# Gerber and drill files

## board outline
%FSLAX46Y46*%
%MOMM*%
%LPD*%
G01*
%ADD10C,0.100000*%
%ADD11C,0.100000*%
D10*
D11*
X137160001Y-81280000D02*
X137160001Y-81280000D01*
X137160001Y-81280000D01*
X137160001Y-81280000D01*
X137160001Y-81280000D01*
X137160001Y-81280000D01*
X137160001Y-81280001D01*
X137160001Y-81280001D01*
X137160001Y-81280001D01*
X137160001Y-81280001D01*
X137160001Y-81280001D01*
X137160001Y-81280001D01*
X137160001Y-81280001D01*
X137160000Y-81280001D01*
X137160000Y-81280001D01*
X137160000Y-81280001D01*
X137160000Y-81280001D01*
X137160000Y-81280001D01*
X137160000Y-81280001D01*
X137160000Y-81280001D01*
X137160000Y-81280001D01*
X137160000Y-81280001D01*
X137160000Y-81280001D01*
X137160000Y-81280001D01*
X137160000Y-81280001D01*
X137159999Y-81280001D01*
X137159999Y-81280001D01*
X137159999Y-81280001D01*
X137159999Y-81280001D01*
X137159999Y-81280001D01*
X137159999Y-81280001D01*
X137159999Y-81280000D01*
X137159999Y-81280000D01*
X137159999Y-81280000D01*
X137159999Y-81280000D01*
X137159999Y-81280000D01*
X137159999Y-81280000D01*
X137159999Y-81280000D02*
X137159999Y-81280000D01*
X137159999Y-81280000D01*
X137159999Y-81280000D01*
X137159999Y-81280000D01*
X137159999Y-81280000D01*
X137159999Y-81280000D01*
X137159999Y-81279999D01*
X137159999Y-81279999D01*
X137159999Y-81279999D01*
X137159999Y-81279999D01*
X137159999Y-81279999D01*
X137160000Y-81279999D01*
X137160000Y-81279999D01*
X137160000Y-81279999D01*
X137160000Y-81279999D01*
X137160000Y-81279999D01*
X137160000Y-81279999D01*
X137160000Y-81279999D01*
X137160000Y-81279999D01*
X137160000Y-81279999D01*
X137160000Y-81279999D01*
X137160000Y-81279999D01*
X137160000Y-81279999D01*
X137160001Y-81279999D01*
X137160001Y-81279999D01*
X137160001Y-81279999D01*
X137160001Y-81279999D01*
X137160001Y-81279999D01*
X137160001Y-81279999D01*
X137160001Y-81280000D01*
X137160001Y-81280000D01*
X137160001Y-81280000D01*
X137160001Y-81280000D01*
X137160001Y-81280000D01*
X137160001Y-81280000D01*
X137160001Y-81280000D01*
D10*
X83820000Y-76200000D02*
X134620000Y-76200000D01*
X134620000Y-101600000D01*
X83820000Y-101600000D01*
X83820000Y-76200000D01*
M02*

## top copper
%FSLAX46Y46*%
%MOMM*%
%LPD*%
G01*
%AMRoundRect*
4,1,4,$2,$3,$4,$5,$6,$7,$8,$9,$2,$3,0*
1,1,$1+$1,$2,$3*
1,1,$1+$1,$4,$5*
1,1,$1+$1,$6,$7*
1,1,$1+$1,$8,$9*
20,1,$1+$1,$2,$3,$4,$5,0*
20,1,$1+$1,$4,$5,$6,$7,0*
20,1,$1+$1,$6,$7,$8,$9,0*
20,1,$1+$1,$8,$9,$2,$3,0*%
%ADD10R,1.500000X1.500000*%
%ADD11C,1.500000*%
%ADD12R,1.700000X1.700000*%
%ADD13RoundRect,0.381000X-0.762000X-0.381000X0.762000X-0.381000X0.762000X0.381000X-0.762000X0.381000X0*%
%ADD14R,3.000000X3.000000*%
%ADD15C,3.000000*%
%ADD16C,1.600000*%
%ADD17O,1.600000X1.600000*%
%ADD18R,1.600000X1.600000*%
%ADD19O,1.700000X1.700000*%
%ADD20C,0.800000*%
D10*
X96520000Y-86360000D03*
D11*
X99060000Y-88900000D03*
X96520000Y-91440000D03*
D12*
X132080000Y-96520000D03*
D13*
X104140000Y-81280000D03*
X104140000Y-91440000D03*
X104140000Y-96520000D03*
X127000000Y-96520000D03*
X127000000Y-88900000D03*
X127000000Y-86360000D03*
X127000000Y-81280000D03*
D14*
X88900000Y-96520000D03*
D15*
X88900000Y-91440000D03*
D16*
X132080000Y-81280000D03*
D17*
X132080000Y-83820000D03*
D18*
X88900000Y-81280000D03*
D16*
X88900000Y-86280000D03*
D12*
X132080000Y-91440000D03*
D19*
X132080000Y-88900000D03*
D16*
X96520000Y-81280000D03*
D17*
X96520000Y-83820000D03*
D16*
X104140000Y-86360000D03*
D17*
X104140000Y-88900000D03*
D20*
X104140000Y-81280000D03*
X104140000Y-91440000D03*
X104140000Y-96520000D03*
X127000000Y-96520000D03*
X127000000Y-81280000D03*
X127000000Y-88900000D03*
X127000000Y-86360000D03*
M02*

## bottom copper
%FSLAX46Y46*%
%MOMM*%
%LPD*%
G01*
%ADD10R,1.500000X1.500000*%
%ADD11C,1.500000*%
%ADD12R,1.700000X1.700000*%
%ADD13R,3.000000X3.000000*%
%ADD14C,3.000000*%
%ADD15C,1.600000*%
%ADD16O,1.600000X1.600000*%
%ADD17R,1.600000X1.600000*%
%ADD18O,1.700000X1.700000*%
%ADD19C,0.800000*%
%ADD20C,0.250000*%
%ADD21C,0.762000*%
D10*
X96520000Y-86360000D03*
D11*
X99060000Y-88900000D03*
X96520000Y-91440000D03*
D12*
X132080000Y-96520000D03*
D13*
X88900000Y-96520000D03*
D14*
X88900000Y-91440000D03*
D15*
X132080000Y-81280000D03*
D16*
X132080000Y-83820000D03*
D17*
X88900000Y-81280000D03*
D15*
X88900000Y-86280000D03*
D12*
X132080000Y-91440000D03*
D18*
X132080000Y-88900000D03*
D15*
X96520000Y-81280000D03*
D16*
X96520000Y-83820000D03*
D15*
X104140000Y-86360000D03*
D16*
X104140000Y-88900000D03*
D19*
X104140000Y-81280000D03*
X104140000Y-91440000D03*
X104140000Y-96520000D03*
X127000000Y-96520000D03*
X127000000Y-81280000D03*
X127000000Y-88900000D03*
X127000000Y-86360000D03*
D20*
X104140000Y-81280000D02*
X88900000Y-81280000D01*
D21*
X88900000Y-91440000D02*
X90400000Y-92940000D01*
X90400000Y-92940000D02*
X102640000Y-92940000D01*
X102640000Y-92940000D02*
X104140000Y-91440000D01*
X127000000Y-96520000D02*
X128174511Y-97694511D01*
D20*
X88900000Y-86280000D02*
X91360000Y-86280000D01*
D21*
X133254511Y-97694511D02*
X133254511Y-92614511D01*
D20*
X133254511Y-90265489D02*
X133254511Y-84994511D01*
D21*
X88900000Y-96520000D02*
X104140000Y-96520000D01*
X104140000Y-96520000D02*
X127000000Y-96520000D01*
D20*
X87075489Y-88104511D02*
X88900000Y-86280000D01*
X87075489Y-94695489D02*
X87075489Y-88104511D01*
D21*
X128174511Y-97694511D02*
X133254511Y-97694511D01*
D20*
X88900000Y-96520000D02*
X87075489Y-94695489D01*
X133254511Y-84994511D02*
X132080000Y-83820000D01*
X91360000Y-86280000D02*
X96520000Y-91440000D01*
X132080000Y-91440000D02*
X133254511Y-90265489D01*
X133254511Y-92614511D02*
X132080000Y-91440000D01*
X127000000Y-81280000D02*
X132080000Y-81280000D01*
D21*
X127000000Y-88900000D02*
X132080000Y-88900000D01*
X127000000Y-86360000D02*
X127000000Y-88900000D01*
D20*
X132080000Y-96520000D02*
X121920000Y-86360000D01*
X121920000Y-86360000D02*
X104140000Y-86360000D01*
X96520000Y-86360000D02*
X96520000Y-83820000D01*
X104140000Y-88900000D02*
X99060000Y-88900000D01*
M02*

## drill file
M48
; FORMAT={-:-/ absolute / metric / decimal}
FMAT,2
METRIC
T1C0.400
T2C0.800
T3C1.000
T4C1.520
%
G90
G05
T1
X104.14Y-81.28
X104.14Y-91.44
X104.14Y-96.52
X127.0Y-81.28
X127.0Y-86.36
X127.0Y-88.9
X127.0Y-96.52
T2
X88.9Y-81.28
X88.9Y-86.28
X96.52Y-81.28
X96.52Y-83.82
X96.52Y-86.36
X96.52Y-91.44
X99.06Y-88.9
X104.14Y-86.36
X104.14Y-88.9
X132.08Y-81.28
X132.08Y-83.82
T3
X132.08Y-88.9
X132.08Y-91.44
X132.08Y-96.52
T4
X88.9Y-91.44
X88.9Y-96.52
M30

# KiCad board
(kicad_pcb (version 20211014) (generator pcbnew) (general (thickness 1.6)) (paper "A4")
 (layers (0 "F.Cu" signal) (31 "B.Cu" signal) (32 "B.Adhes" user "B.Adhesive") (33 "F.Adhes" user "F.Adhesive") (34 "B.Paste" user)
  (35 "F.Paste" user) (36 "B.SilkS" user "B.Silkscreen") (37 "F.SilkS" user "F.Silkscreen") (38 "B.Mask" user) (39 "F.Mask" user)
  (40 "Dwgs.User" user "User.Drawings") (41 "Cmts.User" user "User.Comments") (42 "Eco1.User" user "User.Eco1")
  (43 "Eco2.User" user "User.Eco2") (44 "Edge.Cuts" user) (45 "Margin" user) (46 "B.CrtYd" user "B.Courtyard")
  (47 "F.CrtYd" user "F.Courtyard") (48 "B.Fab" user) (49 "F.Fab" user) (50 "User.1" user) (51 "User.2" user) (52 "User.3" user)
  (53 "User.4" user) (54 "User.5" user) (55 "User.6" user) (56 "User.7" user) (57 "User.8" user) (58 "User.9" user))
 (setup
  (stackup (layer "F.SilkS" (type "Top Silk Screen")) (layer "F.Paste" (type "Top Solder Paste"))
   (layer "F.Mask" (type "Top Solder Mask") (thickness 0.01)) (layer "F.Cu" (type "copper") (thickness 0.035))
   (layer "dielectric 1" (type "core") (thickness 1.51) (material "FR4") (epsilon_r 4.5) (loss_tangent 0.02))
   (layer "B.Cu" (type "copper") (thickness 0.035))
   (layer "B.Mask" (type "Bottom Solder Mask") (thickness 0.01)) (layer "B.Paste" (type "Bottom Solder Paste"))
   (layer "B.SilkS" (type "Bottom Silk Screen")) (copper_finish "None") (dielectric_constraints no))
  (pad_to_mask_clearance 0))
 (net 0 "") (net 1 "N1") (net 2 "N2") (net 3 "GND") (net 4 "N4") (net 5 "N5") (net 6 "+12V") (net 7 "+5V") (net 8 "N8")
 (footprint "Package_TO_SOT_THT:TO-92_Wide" (layer "F.Cu") (at 96.52 86.36 -90)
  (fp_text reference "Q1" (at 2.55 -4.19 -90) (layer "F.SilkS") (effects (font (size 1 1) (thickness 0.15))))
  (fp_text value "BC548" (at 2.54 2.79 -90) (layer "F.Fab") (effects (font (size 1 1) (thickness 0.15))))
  (pad "1" thru_hole rect (at 0 0 270) (size 1.5 1.5) (drill 0.8) (layers *.Cu *.Mask) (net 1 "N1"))
  (pad "2" thru_hole circle (at 2.54 -2.54 270) (size 1.5 1.5) (drill 0.8) (layers *.Cu *.Mask) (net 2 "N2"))
  (pad "3" thru_hole circle (at 5.08 0 270) (size 1.5 1.5) (drill 0.8) (layers *.Cu *.Mask) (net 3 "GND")))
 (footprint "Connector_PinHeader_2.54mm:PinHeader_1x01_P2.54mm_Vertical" (layer "F.Cu") (at 132.08 96.52)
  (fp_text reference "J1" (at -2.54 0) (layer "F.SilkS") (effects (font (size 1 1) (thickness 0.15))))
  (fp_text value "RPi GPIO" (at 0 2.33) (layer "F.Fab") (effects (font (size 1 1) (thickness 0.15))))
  (pad "1" thru_hole rect (at 0 0) (size 1.7 1.7) (drill 1) (layers *.Cu *.Mask) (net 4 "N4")))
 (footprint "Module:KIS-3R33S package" (layer "F.Cu") (at 116.84 86.36)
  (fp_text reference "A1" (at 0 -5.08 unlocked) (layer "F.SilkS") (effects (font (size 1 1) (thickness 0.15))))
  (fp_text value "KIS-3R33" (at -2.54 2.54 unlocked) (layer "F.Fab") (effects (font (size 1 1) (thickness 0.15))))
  (pad "1" smd roundrect (at -12.7 -5.08) (size 2.286 1.524) (layers "F.Cu" "F.Paste" "F.Mask") (roundrect_rratio 0.25) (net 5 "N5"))
  (pad "2" smd roundrect (at -12.7 5.08) (size 2.286 1.524) (layers "F.Cu" "F.Paste" "F.Mask") (roundrect_rratio 0.25) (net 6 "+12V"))
  (pad "3" smd roundrect (at -12.7 10.16) (size 2.286 1.524) (layers "F.Cu" "F.Paste" "F.Mask") (roundrect_rratio 0.25) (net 3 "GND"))
  (pad "4" smd roundrect (at 10.16 10.16) (size 2.286 1.524) (layers "F.Cu" "F.Paste" "F.Mask") (roundrect_rratio 0.25) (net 3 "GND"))
  (pad "5" smd roundrect (at 10.16 2.54) (size 2.286 1.524) (layers "F.Cu" "F.Paste" "F.Mask") (roundrect_rratio 0.25) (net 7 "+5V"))
  (pad "6" smd roundrect (at 10.16 0) (size 2.286 1.524) (layers "F.Cu" "F.Paste" "F.Mask") (roundrect_rratio 0.25) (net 7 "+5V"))
  (pad "7" smd roundrect (at 10.16 -5.08) (size 2.286 1.524) (layers "F.Cu" "F.Paste" "F.Mask") (roundrect_rratio 0.25) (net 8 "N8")))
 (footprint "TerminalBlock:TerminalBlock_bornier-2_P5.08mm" (layer "F.Cu") (at 88.9 96.52 90)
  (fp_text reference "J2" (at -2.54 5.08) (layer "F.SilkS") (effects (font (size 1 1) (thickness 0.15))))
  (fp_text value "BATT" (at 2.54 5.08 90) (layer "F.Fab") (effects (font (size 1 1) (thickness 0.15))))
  (pad "1" thru_hole rect (at 0 0 90) (size 3 3) (drill 1.52) (layers *.Cu *.Mask) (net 3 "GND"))
  (pad "2" thru_hole circle (at 5.08 0 90) (size 3 3) (drill 1.52) (layers *.Cu *.Mask) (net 6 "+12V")))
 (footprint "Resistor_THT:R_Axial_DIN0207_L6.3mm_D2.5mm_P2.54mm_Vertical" (layer "F.Cu") (at 132.08 81.28 -90)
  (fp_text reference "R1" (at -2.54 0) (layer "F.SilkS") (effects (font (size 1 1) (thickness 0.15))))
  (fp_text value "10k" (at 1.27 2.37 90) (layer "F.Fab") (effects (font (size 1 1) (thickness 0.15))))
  (pad "1" thru_hole circle (at 0 0 270) (size 1.6 1.6) (drill 0.8) (layers *.Cu *.Mask) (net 8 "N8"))
  (pad "2" thru_hole oval (at 2.54 0 270) (size 1.6 1.6) (drill 0.8) (layers *.Cu *.Mask) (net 3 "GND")))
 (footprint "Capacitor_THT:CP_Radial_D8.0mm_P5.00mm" (layer "F.Cu") (at 88.9 81.28 -90)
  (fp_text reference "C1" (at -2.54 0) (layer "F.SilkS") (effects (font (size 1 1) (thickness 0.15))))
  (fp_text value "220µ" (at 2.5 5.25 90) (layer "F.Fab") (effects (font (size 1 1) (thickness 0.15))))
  (pad "1" thru_hole rect (at 0 0 270) (size 1.6 1.6) (drill 0.8) (layers *.Cu *.Mask) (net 5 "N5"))
  (pad "2" thru_hole circle (at 5 0 270) (size 1.6 1.6) (drill 0.8) (layers *.Cu *.Mask) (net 3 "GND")))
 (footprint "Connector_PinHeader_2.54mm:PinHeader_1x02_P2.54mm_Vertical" (layer "F.Cu") (at 132.08 91.44 180)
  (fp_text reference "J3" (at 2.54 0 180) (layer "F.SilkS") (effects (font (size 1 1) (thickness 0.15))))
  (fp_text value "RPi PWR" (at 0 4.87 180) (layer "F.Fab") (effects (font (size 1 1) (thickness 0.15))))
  (pad "1" thru_hole rect (at 0 0 180) (size 1.7 1.7) (drill 1) (layers *.Cu *.Mask) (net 3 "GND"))
  (pad "2" thru_hole oval (at 0 2.54 180) (size 1.7 1.7) (drill 1) (layers *.Cu *.Mask) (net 7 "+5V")))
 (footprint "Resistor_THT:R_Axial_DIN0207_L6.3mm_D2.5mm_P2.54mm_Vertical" (layer "F.Cu") (at 96.52 81.28 -90)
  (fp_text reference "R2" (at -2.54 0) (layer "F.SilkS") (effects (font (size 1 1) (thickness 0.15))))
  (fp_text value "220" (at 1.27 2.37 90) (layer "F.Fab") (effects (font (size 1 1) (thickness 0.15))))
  (pad "1" thru_hole circle (at 0 0 270) (size 1.6 1.6) (drill 0.8) (layers *.Cu *.Mask) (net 5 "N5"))
  (pad "2" thru_hole oval (at 2.54 0 270) (size 1.6 1.6) (drill 0.8) (layers *.Cu *.Mask) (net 1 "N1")))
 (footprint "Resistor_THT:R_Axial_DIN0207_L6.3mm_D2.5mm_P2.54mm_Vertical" (layer "F.Cu") (at 104.14 86.36 -90)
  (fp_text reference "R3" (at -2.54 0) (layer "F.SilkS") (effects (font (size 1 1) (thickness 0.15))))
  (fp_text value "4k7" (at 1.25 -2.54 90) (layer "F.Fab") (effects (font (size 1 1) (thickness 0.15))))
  (pad "1" thru_hole circle (at 0 0 270) (size 1.6 1.6) (drill 0.8) (layers *.Cu *.Mask) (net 4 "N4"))
  (pad "2" thru_hole oval (at 2.54 0 270) (size 1.6 1.6) (drill 0.8) (layers *.Cu *.Mask) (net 2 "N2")))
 (gr_circle (center 137.16 81.28) (end 137.16 81.28) (layer "Edge.Cuts") (width 0.1) (fill none))
 (gr_rect (start 83.82 76.2) (end 134.62 101.6) (layer "Edge.Cuts") (width 0.1) (fill none))
 (via (at 104.14 81.28) (size 0.8) (drill 0.4) (layers "F.Cu" "B.Cu") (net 5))
 (segment (start 104.14 81.28) (end 88.9 81.28) (width 0.25) (layer "B.Cu") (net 5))
 (via (at 104.14 91.44) (size 0.8) (drill 0.4) (layers "F.Cu" "B.Cu") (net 6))
 (segment (start 88.9 91.44) (end 90.4 92.94) (width 0.762) (layer "B.Cu") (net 6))
 (segment (start 90.4 92.94) (end 102.64 92.94) (width 0.762) (layer "B.Cu") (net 6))
 (segment (start 102.64 92.94) (end 104.14 91.44) (width 0.762) (layer "B.Cu") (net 6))
 (via (at 104.14 96.52) (size 0.8) (drill 0.4) (layers "F.Cu" "B.Cu") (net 3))
 (via (at 127 96.52) (size 0.8) (drill 0.4) (layers "F.Cu" "B.Cu") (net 3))
 (segment (start 127 96.52) (end 128.174511 97.694511) (width 0.762) (layer "B.Cu") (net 3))
 (segment (start 88.9 86.28) (end 91.36 86.28) (width 0.25) (layer "B.Cu") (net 3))
 (segment (start 133.254511 97.694511) (end 133.254511 92.614511) (width 0.762) (layer "B.Cu") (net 3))
 (segment (start 133.254511 90.265489) (end 133.254511 84.994511) (width 0.25) (layer "B.Cu") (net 3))
 (segment (start 88.9 96.52) (end 104.14 96.52) (width 0.762) (layer "B.Cu") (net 3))
 (segment (start 104.14 96.52) (end 127 96.52) (width 0.762) (layer "B.Cu") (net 3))
 (segment (start 87.075489 88.104511) (end 88.9 86.28) (width 0.25) (layer "B.Cu") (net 3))
 (segment (start 87.075489 94.695489) (end 87.075489 88.104511) (width 0.25) (layer "B.Cu") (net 3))
 (segment (start 128.174511 97.694511) (end 133.254511 97.694511) (width 0.762) (layer "B.Cu") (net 3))
 (segment (start 88.9 96.52) (end 87.075489 94.695489) (width 0.25) (layer "B.Cu") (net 3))
 (segment (start 133.254511 84.994511) (end 132.08 83.82) (width 0.25) (layer "B.Cu") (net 3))
 (segment (start 91.36 86.28) (end 96.52 91.44) (width 0.25) (layer "B.Cu") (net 3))
 (segment (start 132.08 91.44) (end 133.254511 90.265489) (width 0.25) (layer "B.Cu") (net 3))
 (segment (start 133.254511 92.614511) (end 132.08 91.44) (width 0.25) (layer "B.Cu") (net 3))
 (via (at 127 81.28) (size 0.8) (drill 0.4) (layers "F.Cu" "B.Cu") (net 8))
 (segment (start 127 81.28) (end 132.08 81.28) (width 0.25) (layer "B.Cu") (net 8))
 (via (at 127 88.9) (size 0.8) (drill 0.4) (layers "F.Cu" "B.Cu") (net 7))
 (via (at 127 86.36) (size 0.8) (drill 0.4) (layers "F.Cu" "B.Cu") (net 7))
 (segment (start 127 88.9) (end 132.08 88.9) (width 0.762) (layer "B.Cu") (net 7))
 (segment (start 127 86.36) (end 127 88.9) (width 0.762) (layer "B.Cu") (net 7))
 (segment (start 132.08 96.52) (end 121.92 86.36) (width 0.25) (layer "B.Cu") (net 4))
 (segment (start 121.92 86.36) (end 104.14 86.36) (width 0.25) (layer "B.Cu") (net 4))
 (segment (start 96.52 86.36) (end 96.52 83.82) (width 0.25) (layer "B.Cu") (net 1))
 (segment (start 104.14 88.9) (end 99.06 88.9) (width 0.25) (layer "B.Cu") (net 2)))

